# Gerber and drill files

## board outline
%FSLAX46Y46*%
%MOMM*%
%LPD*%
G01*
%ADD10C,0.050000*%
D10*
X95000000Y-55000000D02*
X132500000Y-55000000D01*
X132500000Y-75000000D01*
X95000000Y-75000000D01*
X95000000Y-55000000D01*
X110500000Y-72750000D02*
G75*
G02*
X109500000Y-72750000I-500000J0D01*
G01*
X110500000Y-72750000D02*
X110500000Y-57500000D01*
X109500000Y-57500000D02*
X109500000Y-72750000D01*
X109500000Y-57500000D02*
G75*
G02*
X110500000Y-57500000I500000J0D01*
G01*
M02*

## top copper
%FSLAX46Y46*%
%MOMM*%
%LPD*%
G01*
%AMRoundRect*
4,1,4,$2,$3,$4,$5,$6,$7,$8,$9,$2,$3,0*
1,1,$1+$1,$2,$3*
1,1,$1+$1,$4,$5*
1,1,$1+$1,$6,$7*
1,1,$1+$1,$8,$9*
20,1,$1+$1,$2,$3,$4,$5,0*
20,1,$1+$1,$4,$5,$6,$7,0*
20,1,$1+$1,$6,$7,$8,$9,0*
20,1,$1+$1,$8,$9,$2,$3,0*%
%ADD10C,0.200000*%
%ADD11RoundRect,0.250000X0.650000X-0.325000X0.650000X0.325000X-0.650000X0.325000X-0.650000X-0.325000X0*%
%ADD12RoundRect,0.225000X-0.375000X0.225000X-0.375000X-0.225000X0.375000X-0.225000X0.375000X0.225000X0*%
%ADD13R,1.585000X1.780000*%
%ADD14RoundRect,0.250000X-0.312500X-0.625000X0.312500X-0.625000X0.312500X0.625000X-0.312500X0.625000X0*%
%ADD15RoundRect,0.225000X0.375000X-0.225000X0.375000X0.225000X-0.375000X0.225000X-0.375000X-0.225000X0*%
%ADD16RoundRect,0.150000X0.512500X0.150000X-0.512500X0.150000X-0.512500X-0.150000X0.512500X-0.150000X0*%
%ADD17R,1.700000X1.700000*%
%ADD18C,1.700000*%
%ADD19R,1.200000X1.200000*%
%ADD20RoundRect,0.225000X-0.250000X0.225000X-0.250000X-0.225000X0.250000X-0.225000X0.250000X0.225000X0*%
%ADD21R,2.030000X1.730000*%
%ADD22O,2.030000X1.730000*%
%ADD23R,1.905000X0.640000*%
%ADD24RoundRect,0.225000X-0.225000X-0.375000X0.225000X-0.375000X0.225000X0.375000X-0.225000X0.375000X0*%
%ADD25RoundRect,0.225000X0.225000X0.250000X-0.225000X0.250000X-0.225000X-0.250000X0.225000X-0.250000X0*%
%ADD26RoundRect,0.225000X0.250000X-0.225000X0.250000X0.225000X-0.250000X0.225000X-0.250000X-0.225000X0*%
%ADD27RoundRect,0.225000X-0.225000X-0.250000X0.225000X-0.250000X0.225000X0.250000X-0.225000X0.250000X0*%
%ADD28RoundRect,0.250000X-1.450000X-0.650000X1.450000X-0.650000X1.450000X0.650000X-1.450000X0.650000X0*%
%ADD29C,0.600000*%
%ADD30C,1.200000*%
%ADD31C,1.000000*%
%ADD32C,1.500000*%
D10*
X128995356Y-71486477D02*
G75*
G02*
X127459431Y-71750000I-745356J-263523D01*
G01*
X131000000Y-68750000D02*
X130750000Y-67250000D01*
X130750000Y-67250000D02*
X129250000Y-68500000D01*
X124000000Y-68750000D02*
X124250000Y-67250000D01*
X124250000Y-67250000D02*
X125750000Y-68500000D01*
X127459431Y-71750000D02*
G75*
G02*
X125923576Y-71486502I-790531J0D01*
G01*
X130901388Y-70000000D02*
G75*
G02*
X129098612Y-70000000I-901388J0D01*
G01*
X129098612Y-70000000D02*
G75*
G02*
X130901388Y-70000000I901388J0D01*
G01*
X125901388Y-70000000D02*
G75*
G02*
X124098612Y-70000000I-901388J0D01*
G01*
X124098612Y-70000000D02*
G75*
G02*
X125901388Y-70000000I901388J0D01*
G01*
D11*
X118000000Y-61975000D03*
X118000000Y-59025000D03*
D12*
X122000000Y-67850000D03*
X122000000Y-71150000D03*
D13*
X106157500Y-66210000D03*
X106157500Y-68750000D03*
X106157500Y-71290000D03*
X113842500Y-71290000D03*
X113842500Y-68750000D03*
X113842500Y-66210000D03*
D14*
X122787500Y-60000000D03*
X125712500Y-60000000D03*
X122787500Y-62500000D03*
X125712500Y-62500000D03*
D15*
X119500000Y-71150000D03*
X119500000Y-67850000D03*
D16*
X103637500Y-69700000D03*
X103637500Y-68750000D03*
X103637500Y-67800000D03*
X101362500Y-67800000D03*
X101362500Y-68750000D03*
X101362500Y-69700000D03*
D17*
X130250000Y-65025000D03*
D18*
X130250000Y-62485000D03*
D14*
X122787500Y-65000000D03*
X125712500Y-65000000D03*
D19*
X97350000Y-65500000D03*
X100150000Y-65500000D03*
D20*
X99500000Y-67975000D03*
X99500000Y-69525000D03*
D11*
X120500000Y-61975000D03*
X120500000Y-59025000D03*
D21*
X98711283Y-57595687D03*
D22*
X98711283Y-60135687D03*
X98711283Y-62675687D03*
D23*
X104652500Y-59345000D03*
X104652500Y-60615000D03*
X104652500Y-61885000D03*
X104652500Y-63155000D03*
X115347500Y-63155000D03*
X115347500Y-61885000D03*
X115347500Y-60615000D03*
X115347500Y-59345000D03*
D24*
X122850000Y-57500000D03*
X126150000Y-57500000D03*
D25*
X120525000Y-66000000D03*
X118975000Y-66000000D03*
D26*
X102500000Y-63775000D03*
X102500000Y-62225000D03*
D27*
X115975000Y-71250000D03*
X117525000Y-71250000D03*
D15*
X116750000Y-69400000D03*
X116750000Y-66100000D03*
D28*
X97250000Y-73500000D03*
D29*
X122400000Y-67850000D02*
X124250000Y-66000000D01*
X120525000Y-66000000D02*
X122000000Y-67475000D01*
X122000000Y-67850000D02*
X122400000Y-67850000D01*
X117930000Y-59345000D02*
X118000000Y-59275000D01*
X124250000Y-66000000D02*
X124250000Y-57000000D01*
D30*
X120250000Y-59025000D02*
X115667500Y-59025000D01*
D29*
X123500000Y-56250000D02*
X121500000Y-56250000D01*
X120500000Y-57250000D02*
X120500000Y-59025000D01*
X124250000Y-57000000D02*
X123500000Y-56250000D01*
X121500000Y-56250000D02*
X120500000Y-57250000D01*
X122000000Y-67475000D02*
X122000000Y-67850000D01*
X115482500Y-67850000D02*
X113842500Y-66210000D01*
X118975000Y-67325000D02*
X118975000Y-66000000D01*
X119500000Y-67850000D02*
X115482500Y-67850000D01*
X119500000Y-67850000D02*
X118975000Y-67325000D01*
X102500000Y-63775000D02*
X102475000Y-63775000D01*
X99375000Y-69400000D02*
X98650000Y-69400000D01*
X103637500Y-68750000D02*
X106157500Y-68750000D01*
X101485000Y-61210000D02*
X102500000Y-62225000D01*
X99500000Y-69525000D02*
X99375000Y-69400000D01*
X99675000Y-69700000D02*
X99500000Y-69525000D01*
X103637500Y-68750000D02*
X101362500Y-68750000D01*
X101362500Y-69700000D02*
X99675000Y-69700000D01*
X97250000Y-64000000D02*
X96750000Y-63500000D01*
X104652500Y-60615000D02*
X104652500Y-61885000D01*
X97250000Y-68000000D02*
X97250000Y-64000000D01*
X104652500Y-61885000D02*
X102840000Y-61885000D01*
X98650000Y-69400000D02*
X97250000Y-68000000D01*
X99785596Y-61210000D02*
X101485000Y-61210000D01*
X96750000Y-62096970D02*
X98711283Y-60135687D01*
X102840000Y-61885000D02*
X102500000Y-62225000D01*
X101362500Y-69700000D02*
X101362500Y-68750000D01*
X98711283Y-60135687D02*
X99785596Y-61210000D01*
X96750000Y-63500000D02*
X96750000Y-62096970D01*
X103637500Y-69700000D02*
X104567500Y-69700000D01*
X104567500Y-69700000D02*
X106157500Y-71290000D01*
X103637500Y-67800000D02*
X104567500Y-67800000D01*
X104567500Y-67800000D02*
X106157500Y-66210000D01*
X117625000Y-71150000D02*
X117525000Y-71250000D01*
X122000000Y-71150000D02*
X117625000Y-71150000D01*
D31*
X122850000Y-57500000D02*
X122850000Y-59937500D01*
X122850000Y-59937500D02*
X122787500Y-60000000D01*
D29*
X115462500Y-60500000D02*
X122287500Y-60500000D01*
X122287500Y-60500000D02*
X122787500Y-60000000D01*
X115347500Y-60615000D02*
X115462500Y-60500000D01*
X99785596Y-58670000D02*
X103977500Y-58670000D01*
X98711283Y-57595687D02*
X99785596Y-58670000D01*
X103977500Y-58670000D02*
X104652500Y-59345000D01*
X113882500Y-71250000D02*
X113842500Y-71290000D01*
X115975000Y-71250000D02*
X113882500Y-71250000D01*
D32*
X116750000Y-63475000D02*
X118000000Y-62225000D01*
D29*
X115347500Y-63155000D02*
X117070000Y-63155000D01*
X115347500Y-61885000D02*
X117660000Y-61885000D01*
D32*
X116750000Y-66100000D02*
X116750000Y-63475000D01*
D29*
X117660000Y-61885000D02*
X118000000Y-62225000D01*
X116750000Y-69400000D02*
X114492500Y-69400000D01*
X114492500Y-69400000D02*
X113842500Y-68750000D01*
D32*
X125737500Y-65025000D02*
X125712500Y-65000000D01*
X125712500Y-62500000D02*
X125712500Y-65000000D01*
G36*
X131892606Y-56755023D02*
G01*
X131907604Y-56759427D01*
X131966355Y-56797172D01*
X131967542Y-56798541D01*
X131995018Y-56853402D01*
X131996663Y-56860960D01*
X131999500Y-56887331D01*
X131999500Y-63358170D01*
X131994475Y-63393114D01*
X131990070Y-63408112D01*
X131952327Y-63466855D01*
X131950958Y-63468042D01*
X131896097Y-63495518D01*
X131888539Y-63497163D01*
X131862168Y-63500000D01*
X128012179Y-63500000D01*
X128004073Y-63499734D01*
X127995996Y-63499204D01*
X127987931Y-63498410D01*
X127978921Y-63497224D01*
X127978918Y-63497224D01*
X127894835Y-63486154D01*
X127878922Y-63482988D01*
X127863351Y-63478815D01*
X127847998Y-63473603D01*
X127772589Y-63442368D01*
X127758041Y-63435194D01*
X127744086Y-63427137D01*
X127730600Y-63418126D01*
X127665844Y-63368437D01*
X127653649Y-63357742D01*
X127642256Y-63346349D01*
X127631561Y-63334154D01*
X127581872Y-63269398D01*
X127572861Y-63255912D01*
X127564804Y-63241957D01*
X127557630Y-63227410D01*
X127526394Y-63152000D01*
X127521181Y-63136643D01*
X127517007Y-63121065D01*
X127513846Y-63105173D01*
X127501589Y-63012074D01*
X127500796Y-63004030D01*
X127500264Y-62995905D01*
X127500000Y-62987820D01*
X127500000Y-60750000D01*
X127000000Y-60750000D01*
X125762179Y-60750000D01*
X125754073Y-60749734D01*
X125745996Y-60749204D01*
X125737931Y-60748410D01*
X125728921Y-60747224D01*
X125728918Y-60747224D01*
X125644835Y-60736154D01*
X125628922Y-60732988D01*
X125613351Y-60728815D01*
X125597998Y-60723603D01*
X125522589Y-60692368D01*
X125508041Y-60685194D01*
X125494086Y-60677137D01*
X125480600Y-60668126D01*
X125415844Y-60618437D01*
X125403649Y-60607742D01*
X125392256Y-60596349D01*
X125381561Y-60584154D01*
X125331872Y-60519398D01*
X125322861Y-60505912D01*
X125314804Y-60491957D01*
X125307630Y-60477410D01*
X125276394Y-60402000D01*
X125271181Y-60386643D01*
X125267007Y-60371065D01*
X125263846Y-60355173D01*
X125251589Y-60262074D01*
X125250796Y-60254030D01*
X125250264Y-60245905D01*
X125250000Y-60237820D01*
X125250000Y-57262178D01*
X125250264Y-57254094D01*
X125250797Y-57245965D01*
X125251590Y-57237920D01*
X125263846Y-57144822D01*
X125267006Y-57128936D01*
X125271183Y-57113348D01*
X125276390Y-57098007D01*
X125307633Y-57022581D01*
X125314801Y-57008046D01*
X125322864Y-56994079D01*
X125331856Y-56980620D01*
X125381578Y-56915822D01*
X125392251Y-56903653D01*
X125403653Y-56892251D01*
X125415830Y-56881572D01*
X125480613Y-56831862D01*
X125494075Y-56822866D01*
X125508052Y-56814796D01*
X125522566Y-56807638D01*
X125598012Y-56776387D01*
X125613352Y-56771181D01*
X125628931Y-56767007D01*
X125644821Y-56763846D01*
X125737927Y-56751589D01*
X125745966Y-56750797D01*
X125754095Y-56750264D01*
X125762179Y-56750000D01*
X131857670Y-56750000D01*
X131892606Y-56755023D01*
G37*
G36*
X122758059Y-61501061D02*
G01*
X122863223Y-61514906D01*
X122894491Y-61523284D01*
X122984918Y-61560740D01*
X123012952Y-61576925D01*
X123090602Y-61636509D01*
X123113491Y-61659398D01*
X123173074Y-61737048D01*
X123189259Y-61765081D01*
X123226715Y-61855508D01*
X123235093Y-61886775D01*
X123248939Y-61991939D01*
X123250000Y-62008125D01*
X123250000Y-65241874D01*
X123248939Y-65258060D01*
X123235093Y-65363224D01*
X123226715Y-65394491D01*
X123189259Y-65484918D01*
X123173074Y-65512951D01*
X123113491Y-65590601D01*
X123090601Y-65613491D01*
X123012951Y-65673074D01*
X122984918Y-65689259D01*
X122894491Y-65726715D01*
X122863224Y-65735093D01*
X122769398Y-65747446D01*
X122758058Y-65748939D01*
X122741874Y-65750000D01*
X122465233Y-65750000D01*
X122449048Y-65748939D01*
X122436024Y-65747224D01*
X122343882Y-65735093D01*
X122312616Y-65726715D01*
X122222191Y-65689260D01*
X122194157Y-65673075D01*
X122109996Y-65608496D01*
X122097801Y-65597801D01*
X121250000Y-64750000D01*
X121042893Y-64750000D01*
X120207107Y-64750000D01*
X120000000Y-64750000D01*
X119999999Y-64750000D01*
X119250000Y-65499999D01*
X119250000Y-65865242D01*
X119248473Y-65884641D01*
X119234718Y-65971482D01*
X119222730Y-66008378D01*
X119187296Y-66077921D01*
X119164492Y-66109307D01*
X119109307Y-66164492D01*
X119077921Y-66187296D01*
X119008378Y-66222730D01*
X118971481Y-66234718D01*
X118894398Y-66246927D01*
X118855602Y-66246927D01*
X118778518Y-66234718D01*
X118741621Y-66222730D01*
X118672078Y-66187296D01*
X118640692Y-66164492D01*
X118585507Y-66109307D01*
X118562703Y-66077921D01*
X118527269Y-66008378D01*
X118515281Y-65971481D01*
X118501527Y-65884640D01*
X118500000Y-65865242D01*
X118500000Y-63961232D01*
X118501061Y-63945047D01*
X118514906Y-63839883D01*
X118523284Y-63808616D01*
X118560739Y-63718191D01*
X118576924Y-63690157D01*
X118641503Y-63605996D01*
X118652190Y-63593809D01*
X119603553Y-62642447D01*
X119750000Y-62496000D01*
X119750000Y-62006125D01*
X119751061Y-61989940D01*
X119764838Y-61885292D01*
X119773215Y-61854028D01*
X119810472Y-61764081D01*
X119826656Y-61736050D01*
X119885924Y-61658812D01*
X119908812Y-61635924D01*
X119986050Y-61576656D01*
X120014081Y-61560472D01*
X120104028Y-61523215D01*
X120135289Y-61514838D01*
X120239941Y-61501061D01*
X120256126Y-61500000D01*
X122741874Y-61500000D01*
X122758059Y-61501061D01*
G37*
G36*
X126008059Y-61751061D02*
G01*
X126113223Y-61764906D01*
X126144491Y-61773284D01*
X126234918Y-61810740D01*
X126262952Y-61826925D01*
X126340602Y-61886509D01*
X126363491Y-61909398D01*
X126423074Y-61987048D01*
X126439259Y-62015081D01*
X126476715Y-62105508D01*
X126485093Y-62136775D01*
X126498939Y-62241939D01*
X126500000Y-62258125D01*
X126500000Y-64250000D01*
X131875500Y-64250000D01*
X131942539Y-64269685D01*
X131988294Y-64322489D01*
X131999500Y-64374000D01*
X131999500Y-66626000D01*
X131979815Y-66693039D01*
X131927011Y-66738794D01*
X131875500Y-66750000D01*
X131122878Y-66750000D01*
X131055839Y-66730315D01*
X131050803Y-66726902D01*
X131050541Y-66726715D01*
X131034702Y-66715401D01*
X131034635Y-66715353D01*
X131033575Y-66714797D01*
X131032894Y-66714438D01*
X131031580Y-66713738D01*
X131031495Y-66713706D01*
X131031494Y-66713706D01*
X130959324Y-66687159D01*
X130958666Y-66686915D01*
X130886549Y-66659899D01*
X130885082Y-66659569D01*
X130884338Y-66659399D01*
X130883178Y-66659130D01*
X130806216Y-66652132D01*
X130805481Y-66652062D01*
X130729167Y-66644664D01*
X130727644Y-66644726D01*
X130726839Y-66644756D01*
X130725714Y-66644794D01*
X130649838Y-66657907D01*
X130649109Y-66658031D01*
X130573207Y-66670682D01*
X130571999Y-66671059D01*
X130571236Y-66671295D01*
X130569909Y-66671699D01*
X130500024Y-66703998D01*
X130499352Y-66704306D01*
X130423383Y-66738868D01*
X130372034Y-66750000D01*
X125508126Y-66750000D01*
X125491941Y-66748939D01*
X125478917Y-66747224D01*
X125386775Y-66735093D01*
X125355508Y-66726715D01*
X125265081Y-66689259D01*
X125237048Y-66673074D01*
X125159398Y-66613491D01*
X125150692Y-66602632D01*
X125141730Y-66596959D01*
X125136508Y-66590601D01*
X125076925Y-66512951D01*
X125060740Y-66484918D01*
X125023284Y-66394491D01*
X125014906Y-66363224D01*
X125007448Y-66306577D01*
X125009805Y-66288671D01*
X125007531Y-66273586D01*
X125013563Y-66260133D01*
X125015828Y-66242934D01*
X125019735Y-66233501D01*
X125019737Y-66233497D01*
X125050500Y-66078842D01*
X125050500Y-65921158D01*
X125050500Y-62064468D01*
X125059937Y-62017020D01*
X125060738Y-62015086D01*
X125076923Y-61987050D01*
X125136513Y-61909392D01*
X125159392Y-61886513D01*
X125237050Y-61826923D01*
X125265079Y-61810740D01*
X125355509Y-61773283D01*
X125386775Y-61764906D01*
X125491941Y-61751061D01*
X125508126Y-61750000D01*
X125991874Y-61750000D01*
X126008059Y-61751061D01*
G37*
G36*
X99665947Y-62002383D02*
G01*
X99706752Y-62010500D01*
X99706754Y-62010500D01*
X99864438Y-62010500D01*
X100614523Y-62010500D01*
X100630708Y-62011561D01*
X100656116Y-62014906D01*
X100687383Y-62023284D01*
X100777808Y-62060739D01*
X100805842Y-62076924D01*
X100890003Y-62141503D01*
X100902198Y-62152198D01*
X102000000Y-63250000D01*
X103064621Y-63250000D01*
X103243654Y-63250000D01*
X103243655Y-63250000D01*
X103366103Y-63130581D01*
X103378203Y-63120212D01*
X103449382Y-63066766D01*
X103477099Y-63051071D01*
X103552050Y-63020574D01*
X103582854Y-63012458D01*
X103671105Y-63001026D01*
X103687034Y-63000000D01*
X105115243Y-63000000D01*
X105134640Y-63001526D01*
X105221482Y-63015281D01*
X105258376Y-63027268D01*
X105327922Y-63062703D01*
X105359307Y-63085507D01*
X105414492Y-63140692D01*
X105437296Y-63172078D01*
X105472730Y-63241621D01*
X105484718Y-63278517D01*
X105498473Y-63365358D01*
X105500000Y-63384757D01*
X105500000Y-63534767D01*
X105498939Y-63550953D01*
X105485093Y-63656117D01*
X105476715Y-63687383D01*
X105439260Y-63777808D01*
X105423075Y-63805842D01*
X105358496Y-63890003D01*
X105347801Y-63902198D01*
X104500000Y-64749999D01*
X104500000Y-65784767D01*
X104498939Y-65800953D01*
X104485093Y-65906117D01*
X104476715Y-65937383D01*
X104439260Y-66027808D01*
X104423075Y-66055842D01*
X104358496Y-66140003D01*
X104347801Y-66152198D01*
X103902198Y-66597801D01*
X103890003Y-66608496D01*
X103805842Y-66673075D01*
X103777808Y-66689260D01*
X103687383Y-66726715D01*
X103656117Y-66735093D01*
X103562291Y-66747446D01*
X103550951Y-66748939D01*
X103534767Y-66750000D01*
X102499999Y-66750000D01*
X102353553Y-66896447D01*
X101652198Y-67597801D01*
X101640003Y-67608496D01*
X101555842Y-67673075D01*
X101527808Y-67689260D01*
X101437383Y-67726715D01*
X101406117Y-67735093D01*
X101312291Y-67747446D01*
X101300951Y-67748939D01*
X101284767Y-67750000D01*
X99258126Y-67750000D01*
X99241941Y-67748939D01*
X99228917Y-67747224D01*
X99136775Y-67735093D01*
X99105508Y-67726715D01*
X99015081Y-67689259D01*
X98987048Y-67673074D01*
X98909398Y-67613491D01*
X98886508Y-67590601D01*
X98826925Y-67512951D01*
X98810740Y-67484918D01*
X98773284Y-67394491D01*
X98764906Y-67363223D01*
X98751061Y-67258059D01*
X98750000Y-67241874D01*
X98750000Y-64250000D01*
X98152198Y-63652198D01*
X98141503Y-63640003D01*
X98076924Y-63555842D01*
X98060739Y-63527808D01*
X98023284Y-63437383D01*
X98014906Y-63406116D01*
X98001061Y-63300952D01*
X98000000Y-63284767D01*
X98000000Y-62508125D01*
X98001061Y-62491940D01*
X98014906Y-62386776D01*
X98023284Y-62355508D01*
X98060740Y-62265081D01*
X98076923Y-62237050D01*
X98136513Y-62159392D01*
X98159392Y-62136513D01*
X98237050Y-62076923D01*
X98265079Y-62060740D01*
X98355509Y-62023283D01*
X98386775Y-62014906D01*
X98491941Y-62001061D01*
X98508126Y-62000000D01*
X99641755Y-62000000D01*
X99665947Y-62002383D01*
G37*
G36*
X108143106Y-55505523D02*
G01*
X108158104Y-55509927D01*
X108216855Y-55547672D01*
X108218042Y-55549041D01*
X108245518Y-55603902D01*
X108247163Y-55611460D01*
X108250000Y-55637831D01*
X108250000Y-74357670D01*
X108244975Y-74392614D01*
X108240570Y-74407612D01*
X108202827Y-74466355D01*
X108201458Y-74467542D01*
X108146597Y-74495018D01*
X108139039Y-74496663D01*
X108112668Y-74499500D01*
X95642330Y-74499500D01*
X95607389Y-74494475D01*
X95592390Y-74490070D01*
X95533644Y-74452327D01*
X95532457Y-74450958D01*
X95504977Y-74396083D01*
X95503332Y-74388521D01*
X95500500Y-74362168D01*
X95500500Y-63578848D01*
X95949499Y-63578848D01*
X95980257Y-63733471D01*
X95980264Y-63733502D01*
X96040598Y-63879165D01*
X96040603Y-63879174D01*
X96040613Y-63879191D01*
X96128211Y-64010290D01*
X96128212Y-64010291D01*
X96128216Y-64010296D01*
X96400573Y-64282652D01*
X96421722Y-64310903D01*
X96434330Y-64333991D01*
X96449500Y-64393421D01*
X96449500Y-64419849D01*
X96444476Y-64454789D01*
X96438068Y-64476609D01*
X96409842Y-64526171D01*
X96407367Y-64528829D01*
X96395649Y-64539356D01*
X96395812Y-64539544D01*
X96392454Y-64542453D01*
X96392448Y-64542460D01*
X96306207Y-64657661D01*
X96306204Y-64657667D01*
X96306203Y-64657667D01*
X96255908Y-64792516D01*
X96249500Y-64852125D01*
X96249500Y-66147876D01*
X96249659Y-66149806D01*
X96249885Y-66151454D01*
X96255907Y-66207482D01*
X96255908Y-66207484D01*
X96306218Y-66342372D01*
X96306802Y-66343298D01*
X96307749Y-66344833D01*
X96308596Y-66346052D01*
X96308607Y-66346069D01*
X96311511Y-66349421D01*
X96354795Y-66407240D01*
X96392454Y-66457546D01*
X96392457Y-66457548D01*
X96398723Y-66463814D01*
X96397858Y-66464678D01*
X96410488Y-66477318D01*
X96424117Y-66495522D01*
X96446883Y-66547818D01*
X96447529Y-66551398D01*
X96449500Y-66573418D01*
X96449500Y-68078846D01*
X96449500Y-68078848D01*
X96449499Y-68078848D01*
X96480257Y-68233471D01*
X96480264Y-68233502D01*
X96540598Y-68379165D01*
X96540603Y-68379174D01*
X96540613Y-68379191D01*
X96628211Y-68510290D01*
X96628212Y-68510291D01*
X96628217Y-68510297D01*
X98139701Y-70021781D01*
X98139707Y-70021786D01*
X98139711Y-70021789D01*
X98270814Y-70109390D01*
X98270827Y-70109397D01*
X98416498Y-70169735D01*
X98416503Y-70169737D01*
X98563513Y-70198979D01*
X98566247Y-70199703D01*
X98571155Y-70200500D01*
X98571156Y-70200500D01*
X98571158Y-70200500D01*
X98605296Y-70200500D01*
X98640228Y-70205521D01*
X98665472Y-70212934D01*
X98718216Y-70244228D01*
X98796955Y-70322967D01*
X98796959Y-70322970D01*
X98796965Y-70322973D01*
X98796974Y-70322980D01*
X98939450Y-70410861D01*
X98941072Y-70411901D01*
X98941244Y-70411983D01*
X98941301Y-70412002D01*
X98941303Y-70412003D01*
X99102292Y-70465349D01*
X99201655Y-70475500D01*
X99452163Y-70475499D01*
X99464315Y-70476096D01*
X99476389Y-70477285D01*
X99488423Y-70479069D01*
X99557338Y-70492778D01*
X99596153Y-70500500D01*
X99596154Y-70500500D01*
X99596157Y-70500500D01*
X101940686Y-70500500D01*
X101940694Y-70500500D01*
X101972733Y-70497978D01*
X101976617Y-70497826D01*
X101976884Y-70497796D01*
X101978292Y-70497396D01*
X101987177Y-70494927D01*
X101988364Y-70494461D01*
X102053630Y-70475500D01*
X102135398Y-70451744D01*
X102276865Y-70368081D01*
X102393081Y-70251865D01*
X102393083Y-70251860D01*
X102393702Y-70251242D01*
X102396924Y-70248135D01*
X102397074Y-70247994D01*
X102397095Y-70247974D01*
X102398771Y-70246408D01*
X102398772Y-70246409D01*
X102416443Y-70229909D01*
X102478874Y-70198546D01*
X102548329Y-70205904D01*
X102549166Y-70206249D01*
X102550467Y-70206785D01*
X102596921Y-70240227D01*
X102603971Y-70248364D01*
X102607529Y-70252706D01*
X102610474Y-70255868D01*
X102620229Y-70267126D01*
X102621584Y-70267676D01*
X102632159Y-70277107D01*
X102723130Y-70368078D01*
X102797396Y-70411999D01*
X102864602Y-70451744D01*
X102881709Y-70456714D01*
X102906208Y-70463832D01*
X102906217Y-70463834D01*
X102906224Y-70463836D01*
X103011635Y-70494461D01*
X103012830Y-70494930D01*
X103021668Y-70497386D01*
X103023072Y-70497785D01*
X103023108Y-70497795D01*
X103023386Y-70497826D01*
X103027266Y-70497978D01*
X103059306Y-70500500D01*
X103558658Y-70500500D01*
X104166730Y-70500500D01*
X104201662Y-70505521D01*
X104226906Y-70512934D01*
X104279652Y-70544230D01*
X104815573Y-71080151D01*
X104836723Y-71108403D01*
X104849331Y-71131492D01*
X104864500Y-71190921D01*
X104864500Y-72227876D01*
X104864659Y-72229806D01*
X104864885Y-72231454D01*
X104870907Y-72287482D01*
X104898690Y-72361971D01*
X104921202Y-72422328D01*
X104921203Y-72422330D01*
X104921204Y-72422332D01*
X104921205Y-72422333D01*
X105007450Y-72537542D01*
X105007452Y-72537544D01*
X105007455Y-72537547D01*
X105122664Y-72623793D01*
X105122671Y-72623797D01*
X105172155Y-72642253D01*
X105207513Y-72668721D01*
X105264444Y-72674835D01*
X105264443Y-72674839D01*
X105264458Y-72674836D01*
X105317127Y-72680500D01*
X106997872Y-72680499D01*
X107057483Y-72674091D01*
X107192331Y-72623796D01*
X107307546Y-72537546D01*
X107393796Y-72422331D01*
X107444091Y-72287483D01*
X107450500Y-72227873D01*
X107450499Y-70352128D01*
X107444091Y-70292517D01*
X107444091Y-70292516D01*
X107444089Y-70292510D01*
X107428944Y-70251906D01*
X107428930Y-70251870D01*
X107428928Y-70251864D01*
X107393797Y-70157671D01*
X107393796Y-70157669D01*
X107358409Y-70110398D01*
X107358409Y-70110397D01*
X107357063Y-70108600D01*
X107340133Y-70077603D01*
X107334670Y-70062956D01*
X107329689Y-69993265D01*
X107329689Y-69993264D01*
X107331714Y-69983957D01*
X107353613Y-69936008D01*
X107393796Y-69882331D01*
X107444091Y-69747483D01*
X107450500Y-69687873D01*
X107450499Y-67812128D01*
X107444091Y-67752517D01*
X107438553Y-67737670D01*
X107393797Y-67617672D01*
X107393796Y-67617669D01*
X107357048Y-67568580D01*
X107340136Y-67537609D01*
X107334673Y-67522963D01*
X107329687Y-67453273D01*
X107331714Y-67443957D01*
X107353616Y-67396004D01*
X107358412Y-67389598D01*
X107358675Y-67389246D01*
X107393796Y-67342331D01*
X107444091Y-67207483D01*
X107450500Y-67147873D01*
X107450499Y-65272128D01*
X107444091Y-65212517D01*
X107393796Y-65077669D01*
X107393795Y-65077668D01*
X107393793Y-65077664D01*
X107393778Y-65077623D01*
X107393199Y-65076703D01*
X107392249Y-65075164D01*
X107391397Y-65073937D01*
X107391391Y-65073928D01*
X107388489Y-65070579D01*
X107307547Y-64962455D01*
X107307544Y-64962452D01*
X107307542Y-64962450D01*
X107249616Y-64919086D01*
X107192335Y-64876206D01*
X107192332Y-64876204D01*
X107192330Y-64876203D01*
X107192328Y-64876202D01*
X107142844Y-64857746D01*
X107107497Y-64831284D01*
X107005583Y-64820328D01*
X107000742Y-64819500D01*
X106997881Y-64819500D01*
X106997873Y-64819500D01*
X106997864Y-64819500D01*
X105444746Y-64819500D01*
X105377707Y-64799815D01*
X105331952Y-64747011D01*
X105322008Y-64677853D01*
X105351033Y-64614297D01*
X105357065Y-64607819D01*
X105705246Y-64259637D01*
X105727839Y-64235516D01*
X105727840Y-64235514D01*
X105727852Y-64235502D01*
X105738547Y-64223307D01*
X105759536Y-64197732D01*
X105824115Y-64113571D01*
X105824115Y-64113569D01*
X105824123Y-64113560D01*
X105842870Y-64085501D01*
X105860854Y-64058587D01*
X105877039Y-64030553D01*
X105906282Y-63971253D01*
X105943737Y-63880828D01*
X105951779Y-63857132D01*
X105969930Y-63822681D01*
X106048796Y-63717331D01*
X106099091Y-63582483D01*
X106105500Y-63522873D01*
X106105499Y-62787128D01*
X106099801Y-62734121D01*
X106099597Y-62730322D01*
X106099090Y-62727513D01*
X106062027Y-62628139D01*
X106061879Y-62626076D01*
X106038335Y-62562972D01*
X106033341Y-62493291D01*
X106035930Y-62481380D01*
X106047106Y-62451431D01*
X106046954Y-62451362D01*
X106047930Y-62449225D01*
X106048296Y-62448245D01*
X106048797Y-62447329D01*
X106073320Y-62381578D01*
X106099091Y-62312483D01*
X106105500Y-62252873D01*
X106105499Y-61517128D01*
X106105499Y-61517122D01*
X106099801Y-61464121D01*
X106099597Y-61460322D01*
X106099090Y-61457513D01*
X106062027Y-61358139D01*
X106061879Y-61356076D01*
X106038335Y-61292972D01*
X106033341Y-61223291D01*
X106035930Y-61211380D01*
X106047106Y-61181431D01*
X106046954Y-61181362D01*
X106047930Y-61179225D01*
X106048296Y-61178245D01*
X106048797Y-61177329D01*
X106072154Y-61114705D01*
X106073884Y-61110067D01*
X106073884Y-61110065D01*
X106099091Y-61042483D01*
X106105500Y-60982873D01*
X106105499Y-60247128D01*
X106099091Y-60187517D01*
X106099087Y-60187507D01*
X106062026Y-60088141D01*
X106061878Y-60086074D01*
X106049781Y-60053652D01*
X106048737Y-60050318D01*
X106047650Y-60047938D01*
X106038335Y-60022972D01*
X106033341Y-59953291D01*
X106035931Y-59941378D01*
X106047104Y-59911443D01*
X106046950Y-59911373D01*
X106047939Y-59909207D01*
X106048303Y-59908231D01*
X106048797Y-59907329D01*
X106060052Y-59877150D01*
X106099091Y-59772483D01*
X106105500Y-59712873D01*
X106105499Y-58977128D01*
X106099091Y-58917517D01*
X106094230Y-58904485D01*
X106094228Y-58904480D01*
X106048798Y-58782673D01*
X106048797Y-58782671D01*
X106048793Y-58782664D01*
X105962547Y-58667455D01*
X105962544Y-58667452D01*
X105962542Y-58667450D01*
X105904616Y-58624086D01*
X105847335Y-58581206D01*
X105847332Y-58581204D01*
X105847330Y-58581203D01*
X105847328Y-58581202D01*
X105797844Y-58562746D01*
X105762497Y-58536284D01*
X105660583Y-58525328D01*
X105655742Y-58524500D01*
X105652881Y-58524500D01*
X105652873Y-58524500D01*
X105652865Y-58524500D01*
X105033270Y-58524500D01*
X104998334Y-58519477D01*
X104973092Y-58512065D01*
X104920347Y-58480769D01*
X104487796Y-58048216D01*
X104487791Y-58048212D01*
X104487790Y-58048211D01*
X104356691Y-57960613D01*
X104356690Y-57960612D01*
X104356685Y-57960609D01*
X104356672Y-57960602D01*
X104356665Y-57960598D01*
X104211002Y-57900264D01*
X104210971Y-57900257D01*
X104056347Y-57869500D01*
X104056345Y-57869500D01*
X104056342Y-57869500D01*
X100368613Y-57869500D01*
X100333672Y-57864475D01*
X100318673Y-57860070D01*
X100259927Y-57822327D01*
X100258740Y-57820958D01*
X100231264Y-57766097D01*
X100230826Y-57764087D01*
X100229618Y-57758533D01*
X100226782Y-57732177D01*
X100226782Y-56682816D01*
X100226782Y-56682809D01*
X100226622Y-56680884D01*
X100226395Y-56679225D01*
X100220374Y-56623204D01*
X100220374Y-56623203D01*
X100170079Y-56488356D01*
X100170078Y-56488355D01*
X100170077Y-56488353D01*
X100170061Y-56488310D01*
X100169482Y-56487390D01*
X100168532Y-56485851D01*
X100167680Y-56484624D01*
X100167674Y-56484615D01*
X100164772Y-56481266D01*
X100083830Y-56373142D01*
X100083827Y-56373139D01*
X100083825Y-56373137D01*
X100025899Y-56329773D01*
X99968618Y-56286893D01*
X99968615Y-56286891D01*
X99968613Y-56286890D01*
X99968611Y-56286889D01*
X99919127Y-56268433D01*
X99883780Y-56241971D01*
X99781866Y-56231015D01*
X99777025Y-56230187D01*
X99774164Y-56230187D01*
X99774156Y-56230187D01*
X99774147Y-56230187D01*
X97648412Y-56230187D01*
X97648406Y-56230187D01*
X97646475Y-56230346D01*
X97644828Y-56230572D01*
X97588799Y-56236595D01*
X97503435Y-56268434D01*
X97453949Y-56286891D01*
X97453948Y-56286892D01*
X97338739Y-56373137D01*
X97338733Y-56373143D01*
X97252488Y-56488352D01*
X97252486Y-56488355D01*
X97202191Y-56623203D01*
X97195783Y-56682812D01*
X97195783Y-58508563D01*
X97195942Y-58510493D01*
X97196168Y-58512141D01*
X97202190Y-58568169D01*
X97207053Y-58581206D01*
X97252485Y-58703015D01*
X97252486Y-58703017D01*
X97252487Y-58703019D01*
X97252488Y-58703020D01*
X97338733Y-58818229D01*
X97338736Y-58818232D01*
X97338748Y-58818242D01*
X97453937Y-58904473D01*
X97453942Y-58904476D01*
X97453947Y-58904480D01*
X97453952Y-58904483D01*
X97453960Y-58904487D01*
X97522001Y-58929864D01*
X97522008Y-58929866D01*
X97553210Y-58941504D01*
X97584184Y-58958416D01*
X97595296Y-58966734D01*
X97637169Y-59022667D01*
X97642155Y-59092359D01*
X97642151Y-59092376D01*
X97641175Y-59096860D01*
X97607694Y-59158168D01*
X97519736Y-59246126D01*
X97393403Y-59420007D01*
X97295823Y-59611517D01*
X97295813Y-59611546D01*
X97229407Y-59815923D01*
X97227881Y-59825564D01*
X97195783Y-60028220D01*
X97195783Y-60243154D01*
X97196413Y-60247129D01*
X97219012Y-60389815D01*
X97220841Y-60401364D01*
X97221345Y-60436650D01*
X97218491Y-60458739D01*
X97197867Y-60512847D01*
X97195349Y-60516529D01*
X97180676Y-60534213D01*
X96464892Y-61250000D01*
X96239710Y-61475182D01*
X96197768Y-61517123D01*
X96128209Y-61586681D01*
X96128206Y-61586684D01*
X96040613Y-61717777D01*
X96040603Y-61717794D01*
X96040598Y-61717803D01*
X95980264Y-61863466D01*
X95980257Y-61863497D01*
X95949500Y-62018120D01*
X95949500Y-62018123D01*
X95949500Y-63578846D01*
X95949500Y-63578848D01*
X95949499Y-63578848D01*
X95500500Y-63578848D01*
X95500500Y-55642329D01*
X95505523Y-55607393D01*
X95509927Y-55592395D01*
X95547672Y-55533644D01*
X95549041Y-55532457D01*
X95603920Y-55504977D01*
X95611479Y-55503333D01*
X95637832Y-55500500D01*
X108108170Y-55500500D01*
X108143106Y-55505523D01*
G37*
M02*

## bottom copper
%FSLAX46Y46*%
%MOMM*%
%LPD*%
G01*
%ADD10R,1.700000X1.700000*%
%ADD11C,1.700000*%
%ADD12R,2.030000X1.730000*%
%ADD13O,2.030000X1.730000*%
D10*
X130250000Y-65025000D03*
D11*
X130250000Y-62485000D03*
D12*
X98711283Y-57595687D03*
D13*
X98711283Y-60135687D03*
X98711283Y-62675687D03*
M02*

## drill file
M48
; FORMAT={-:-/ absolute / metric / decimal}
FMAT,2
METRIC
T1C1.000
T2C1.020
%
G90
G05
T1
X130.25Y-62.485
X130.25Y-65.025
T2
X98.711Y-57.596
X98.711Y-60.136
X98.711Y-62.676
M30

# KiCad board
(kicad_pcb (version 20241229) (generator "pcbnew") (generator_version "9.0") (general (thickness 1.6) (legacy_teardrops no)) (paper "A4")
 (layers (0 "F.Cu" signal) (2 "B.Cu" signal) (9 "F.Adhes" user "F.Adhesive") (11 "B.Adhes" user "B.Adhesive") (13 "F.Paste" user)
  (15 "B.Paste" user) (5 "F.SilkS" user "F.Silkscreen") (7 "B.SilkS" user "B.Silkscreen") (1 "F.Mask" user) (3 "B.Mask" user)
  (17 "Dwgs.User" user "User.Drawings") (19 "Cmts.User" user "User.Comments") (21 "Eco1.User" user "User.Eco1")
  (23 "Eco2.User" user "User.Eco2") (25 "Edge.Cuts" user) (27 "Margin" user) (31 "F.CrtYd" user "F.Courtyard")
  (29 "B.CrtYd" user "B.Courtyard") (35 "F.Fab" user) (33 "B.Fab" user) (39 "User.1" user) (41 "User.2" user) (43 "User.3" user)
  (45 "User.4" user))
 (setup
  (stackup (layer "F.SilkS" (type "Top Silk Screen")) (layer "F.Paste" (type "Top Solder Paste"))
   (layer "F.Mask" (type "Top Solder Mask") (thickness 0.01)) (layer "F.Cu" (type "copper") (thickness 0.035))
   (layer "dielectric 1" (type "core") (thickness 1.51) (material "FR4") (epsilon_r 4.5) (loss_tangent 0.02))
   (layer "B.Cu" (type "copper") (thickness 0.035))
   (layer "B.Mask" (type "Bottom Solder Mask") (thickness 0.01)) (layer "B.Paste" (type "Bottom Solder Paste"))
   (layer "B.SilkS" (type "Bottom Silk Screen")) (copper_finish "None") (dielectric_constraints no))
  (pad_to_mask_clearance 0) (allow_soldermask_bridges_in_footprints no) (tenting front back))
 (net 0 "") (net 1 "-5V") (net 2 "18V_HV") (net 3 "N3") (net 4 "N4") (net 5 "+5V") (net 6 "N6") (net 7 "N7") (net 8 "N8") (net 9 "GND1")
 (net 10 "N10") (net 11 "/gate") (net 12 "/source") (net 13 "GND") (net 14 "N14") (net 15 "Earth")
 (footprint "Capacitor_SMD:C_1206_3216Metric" (layer "F.Cu") (at 118 60.5 90)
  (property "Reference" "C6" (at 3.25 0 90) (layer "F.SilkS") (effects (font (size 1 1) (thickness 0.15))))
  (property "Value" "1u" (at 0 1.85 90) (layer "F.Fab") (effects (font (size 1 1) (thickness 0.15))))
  (pad "1" smd roundrect (at -1.475 0 90) (size 1.15 1.8) (layers "F.Cu" "F.Mask" "F.Paste") (roundrect_rratio 0.217391) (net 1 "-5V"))
  (pad "2" smd roundrect (at 1.475 0 90) (size 1.15 1.8) (layers "F.Cu" "F.Mask" "F.Paste") (roundrect_rratio 0.217391) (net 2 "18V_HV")))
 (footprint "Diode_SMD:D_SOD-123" (layer "F.Cu") (at 122 69.5 -90)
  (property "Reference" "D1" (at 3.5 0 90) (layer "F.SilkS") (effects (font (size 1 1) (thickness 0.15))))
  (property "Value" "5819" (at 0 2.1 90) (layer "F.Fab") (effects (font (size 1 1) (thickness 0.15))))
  (pad "1" smd roundrect (at -1.65 0 270) (size 0.9 1.2) (layers "F.Cu" "F.Mask" "F.Paste") (roundrect_rratio 0.25) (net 2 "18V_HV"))
  (pad "2" smd roundrect (at 1.65 0 270) (size 0.9 1.2) (layers "F.Cu" "F.Mask" "F.Paste") (roundrect_rratio 0.25) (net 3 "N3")))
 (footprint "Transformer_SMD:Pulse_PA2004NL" (layer "F.Cu") (at 110 68.75)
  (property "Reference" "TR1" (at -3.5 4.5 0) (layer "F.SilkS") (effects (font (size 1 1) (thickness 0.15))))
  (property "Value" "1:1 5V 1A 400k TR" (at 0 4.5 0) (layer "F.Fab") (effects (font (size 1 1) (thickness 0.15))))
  (pad "1" smd rect (at -3.8425 -2.54) (size 1.585 1.78) (layers "F.Cu" "F.Mask" "F.Paste") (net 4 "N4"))
  (pad "2" smd rect (at -3.8425 0) (size 1.585 1.78) (layers "F.Cu" "F.Mask" "F.Paste") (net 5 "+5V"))
  (pad "3" smd rect (at -3.8425 2.54) (size 1.585 1.78) (layers "F.Cu" "F.Mask" "F.Paste") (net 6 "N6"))
  (pad "4" smd rect (at 3.8425 2.54) (size 1.585 1.78) (layers "F.Cu" "F.Mask" "F.Paste") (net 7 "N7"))
  (pad "5" smd rect (at 3.8425 0) (size 1.585 1.78) (layers "F.Cu" "F.Mask" "F.Paste") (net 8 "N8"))
  (pad "6" smd rect (at 3.8425 -2.54) (size 1.585 1.78) (layers "F.Cu" "F.Mask" "F.Paste") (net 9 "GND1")))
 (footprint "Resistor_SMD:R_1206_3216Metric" (layer "F.Cu") (at 124.25 60)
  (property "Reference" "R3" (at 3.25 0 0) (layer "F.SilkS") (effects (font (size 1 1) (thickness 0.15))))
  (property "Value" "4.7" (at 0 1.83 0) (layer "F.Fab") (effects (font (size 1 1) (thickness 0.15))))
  (pad "1" smd roundrect (at -1.4625 0) (size 1.125 1.75) (layers "F.Cu" "F.Mask" "F.Paste") (roundrect_rratio 0.222222) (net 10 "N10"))
  (pad "2" smd roundrect (at 1.4625 0) (size 1.125 1.75) (layers "F.Cu" "F.Mask" "F.Paste") (roundrect_rratio 0.222222) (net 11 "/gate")))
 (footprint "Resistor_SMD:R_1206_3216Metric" (layer "F.Cu") (at 124.25 62.5)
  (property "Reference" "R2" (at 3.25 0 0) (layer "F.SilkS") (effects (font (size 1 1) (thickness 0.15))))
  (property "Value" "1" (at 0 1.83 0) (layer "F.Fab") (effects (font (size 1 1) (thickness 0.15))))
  (pad "1" smd roundrect (at -1.4625 0) (size 1.125 1.75) (layers "F.Cu" "F.Mask" "F.Paste") (roundrect_rratio 0.222222) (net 9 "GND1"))
  (pad "2" smd roundrect (at 1.4625 0) (size 1.125 1.75) (layers "F.Cu" "F.Mask" "F.Paste") (roundrect_rratio 0.222222) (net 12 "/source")))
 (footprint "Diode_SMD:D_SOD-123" (layer "F.Cu") (at 119.5 69.5 90)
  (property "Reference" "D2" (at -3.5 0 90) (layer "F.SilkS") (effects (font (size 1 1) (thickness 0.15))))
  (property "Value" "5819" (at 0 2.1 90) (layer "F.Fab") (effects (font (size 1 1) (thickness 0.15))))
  (pad "1" smd roundrect (at -1.65 0 90) (size 0.9 1.2) (layers "F.Cu" "F.Mask" "F.Paste") (roundrect_rratio 0.25) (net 3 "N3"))
  (pad "2" smd roundrect (at 1.65 0 90) (size 0.9 1.2) (layers "F.Cu" "F.Mask" "F.Paste") (roundrect_rratio 0.25) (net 9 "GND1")))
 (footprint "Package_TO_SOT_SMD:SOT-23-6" (layer "F.Cu") (at 102.5 68.75 180)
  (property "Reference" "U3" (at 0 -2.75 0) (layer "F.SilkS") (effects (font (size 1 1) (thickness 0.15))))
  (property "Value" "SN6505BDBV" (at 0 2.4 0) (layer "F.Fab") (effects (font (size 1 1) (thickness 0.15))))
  (pad "1" smd roundrect (at -1.1375 -0.95 180) (size 1.325 0.6) (layers "F.Cu" "F.Mask" "F.Paste") (roundrect_rratio 0.25) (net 6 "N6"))
  (pad "2" smd roundrect (at -1.1375 0 180) (size 1.325 0.6) (layers "F.Cu" "F.Mask" "F.Paste") (roundrect_rratio 0.25) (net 5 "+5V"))
  (pad "3" smd roundrect (at -1.1375 0.95 180) (size 1.325 0.6) (layers "F.Cu" "F.Mask" "F.Paste") (roundrect_rratio 0.25) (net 4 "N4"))
  (pad "4" smd roundrect (at 1.1375 0.95 180) (size 1.325 0.6) (layers "F.Cu" "F.Mask" "F.Paste") (roundrect_rratio 0.25) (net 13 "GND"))
  (pad "5" smd roundrect (at 1.1375 0 180) (size 1.325 0.6) (layers "F.Cu" "F.Mask" "F.Paste") (roundrect_rratio 0.25) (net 5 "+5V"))
  (pad "6" smd roundrect (at 1.1375 -0.95 180) (size 1.325 0.6) (layers "F.Cu" "F.Mask" "F.Paste") (roundrect_rratio 0.25) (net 5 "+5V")))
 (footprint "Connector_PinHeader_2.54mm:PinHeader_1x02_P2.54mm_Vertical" (layer "F.Cu") (at 130.25 65.025 180)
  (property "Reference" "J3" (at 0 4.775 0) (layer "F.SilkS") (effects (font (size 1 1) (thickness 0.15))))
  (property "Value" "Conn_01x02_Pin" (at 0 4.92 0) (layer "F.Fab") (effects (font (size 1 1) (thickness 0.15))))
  (pad "1" thru_hole rect (at 0 0 180) (size 1.7 1.7) (drill 1) (layers "*.Cu" "*.Mask") (remove_unused_layers no) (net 12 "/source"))
  (pad "2" thru_hole circle (at 0 2.54 180) (size 1.7 1.7) (drill 1) (layers "*.Cu" "*.Mask") (remove_unused_layers no) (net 11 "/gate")))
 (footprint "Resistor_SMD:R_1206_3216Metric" (layer "F.Cu") (at 124.25 65)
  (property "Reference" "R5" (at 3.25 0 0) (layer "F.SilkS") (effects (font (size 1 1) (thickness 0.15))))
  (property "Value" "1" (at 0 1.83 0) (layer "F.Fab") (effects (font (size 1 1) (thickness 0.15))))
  (pad "1" smd roundrect (at -1.4625 0) (size 1.125 1.75) (layers "F.Cu" "F.Mask" "F.Paste") (roundrect_rratio 0.222222) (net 9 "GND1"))
  (pad "2" smd roundrect (at 1.4625 0) (size 1.125 1.75) (layers "F.Cu" "F.Mask" "F.Paste") (roundrect_rratio 0.222222) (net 12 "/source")))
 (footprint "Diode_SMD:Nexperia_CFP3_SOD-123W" (layer "F.Cu") (at 98.75 65.5)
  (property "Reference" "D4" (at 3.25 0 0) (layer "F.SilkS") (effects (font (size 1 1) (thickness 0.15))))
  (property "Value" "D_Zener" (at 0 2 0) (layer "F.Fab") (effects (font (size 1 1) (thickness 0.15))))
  (pad "1" smd rect (at -1.4 0) (size 1.2 1.2) (layers "F.Cu" "F.Mask" "F.Paste") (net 5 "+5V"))
  (pad "2" smd rect (at 1.4 0) (size 1.2 1.2) (layers "F.Cu" "F.Mask" "F.Paste") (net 13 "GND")))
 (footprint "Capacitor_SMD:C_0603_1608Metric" (layer "F.Cu") (at 99.5 68.75 -90)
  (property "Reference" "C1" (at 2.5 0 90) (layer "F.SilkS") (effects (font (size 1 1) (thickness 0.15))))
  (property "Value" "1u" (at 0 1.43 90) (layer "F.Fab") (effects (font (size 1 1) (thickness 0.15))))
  (pad "1" smd roundrect (at -0.775 0 270) (size 0.9 0.95) (layers "F.Cu" "F.Mask" "F.Paste") (roundrect_rratio 0.25) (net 13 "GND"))
  (pad "2" smd roundrect (at 0.775 0 270) (size 0.9 0.95) (layers "F.Cu" "F.Mask" "F.Paste") (roundrect_rratio 0.25) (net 5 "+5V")))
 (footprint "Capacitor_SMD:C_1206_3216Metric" (layer "F.Cu") (at 120.5 60.5 90)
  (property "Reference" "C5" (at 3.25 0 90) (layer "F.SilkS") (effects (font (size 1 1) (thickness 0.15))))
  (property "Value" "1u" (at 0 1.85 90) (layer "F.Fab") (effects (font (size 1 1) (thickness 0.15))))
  (pad "1" smd roundrect (at -1.475 0 90) (size 1.15 1.8) (layers "F.Cu" "F.Mask" "F.Paste") (roundrect_rratio 0.217391) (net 9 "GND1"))
  (pad "2" smd roundrect (at 1.475 0 90) (size 1.15 1.8) (layers "F.Cu" "F.Mask" "F.Paste") (roundrect_rratio 0.217391) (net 2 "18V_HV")))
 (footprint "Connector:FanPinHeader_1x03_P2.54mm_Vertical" (layer "F.Cu") (at 98.711283 57.595687 -90)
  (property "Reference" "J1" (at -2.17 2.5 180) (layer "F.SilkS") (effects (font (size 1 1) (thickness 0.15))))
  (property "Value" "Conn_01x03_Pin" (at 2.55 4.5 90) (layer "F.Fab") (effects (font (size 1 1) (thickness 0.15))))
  (pad "1" thru_hole rect (at 0 0) (size 2.03 1.73) (drill 1.02) (layers "*.Cu" "*.Mask") (remove_unused_layers no) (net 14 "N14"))
  (pad "2" thru_hole oval (at 2.54 0) (size 2.03 1.73) (drill 1.02) (layers "*.Cu" "*.Mask") (remove_unused_layers no) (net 5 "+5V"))
  (pad "3" thru_hole oval (at 5.08 0) (size 2.03 1.73) (drill 1.02) (layers "*.Cu" "*.Mask") (remove_unused_layers no) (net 13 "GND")))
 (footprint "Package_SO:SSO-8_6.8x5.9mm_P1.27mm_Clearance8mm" (layer "F.Cu") (at 110 61.25)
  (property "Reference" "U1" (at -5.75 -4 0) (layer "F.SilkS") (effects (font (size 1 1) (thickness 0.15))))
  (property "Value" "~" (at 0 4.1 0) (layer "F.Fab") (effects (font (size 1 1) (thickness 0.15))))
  (pad "1" smd rect (at -5.3475 -1.905) (size 1.905 0.64) (layers "F.Cu" "F.Mask" "F.Paste") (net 14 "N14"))
  (pad "2" smd rect (at -5.3475 -0.635) (size 1.905 0.64) (layers "F.Cu" "F.Mask" "F.Paste") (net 5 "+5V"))
  (pad "3" smd rect (at -5.3475 0.635) (size 1.905 0.64) (layers "F.Cu" "F.Mask" "F.Paste") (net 5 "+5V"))
  (pad "4" smd rect (at -5.3475 1.905) (size 1.905 0.64) (layers "F.Cu" "F.Mask" "F.Paste") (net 13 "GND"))
  (pad "5" smd rect (at 5.3475 1.905) (size 1.905 0.64) (layers "F.Cu" "F.Mask" "F.Paste") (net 1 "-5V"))
  (pad "6" smd rect (at 5.3475 0.635) (size 1.905 0.64) (layers "F.Cu" "F.Mask" "F.Paste") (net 1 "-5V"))
  (pad "7" smd rect (at 5.3475 -0.635) (size 1.905 0.64) (layers "F.Cu" "F.Mask" "F.Paste") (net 10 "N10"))
  (pad "8" smd rect (at 5.3475 -1.905) (size 1.905 0.64) (layers "F.Cu" "F.Mask" "F.Paste") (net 2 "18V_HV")))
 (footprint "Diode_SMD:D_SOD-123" (layer "F.Cu") (at 124.5 57.5)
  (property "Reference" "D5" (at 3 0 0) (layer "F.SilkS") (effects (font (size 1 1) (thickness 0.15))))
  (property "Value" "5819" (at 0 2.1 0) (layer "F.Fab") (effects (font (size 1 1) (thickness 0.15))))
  (pad "1" smd roundrect (at -1.65 0) (size 0.9 1.2) (layers "F.Cu" "F.Mask" "F.Paste") (roundrect_rratio 0.25) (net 10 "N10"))
  (pad "2" smd roundrect (at 1.65 0) (size 0.9 1.2) (layers "F.Cu" "F.Mask" "F.Paste") (roundrect_rratio 0.25) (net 11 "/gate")))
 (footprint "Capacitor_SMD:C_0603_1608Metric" (layer "F.Cu") (at 119.75 66 180)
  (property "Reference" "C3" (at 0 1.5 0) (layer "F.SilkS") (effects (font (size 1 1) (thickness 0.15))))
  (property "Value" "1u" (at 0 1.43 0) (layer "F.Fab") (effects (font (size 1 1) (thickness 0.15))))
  (pad "1" smd roundrect (at -0.775 0 180) (size 0.9 0.95) (layers "F.Cu" "F.Mask" "F.Paste") (roundrect_rratio 0.25) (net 2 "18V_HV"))
  (pad "2" smd roundrect (at 0.775 0 180) (size 0.9 0.95) (layers "F.Cu" "F.Mask" "F.Paste") (roundrect_rratio 0.25) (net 9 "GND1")))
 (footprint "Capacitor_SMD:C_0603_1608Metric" (layer "F.Cu") (at 102.5 63 90)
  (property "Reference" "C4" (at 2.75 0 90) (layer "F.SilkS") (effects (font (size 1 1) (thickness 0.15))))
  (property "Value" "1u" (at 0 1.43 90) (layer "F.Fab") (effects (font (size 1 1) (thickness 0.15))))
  (pad "1" smd roundrect (at -0.775 0 90) (size 0.9 0.95) (layers "F.Cu" "F.Mask" "F.Paste") (roundrect_rratio 0.25) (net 13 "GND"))
  (pad "2" smd roundrect (at 0.775 0 90) (size 0.9 0.95) (layers "F.Cu" "F.Mask" "F.Paste") (roundrect_rratio 0.25) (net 5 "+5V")))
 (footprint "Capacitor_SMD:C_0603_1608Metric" (layer "F.Cu") (at 116.75 71.25)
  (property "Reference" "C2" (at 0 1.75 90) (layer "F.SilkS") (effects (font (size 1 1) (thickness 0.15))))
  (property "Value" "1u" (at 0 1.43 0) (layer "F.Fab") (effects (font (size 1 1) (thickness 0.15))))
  (pad "1" smd roundrect (at -0.775 0) (size 0.9 0.95) (layers "F.Cu" "F.Mask" "F.Paste") (roundrect_rratio 0.25) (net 7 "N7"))
  (pad "2" smd roundrect (at 0.775 0) (size 0.9 0.95) (layers "F.Cu" "F.Mask" "F.Paste") (roundrect_rratio 0.25) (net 3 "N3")))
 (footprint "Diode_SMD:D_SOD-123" (layer "F.Cu") (at 116.75 67.75 90)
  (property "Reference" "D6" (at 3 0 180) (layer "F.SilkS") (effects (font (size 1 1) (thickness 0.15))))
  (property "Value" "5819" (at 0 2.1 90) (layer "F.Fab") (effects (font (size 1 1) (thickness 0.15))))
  (pad "1" smd roundrect (at -1.65 0 90) (size 0.9 1.2) (layers "F.Cu" "F.Mask" "F.Paste") (roundrect_rratio 0.25) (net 8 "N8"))
  (pad "2" smd roundrect (at 1.65 0 90) (size 0.9 1.2) (layers "F.Cu" "F.Mask" "F.Paste") (roundrect_rratio 0.25) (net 1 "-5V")))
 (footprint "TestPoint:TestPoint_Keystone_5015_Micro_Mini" (layer "F.Cu") (at 97.25 73.5)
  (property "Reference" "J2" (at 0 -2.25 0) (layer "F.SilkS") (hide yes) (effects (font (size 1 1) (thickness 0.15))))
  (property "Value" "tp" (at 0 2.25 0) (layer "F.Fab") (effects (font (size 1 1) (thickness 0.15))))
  (pad "1" smd roundrect (at 0 0) (size 3.4 1.8) (layers "F.Cu" "F.Mask" "F.Paste") (roundrect_rratio 0.1388888889) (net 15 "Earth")))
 (gr_arc (start 128.995356 71.486477) (mid 128.383687 72.529184) (end 127.459431 71.75) (stroke (width 0.2) (type default)) (layer "F.Cu"))
 (gr_line (start 131 68.75) (end 130.75 67.25) (stroke (width 0.2) (type default)) (layer "F.Cu"))
 (gr_line (start 130.75 67.25) (end 129.25 68.5) (stroke (width 0.2) (type default)) (layer "F.Cu"))
 (gr_line (start 124 68.75) (end 124.25 67.25) (stroke (width 0.2) (type default)) (layer "F.Cu"))
 (gr_line (start 124.25 67.25) (end 125.75 68.5) (stroke (width 0.2) (type default)) (layer "F.Cu"))
 (gr_arc (start 127.459431 71.75) (mid 126.535175 72.529184) (end 125.923506 71.486477) (stroke (width 0.2) (type default)) (layer "F.Cu"))
 (gr_circle (center 130 70) (end 130.75 70.5) (stroke (width 0.2) (type default)) (fill no) (layer "F.Cu"))
 (gr_circle (center 125 70) (end 125.75 70.5) (stroke (width 0.2) (type default)) (fill no) (layer "F.Cu"))
 (gr_rect (start 95 55) (end 132.5 75) (stroke (width 0.05) (type default)) (fill no) (layer "Edge.Cuts"))
 (gr_arc (start 110.5 72.75) (mid 110 73.25) (end 109.5 72.75) (stroke (width 0.05) (type default)) (layer "Edge.Cuts"))
 (gr_line (start 110.5 72.75) (end 110.5 57.5) (stroke (width 0.05) (type default)) (layer "Edge.Cuts"))
 (gr_line (start 109.5 57.5) (end 109.5 72.75) (stroke (width 0.05) (type default)) (layer "Edge.Cuts"))
 (gr_arc (start 109.5 57.5) (mid 110 57) (end 110.5 57.5) (stroke (width 0.05) (type default)) (layer "Edge.Cuts"))
 (segment (start 122.4 67.85) (end 124.25 66) (width 0.6) (layer "F.Cu") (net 2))
 (segment (start 120.525 66) (end 122 67.475) (width 0.6) (layer "F.Cu") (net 2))
 (segment (start 122 67.85) (end 122.4 67.85) (width 0.6) (layer "F.Cu") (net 2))
 (segment (start 117.93 59.345) (end 118 59.275) (width 0.6) (layer "F.Cu") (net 2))
 (segment (start 124.25 66) (end 124.25 57) (width 0.6) (layer "F.Cu") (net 2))
 (segment (start 120.25 59.025) (end 115.6675 59.025) (width 1.2) (layer "F.Cu") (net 2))
 (segment (start 123.5 56.25) (end 121.5 56.25) (width 0.6) (layer "F.Cu") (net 2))
 (segment (start 120.5 57.25) (end 120.5 59.025) (width 0.6) (layer "F.Cu") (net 2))
 (segment (start 124.25 57) (end 123.5 56.25) (width 0.6) (layer "F.Cu") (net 2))
 (segment (start 121.5 56.25) (end 120.5 57.25) (width 0.6) (layer "F.Cu") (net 2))
 (segment (start 122 67.475) (end 122 67.85) (width 0.6) (layer "F.Cu") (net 2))
 (segment (start 115.4825 67.85) (end 113.8425 66.21) (width 0.6) (layer "F.Cu") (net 9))
 (segment (start 118.975 67.325) (end 118.975 66) (width 0.6) (layer "F.Cu") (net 9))
 (segment (start 119.5 67.85) (end 115.4825 67.85) (width 0.6) (layer "F.Cu") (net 9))
 (segment (start 119.5 67.85) (end 118.975 67.325) (width 0.6) (layer "F.Cu") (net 9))
 (segment (start 102.5 63.775) (end 102.475 63.775) (width 0.6) (layer "F.Cu") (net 13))
 (segment (start 99.375 69.4) (end 98.65 69.4) (width 0.6) (layer "F.Cu") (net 5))
 (segment (start 103.6375 68.75) (end 106.1575 68.75) (width 0.6) (layer "F.Cu") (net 5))
 (segment (start 101.485 61.21) (end 102.5 62.225) (width 0.6) (layer "F.Cu") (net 5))
 (segment (start 99.5 69.525) (end 99.375 69.4) (width 0.6) (layer "F.Cu") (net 5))
 (segment (start 99.675 69.7) (end 99.5 69.525) (width 0.6) (layer "F.Cu") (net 5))
 (segment (start 103.6375 68.75) (end 101.3625 68.75) (width 0.6) (layer "F.Cu") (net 5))
 (segment (start 101.3625 69.7) (end 99.675 69.7) (width 0.6) (layer "F.Cu") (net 5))
 (segment (start 97.25 64) (end 96.75 63.5) (width 0.6) (layer "F.Cu") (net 5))
 (segment (start 104.6525 60.615) (end 104.6525 61.885) (width 0.6) (layer "F.Cu") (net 5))
 (segment (start 97.25 68) (end 97.25 64) (width 0.6) (layer "F.Cu") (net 5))
 (segment (start 104.6525 61.885) (end 102.84 61.885) (width 0.6) (layer "F.Cu") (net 5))
 (segment (start 98.65 69.4) (end 97.25 68) (width 0.6) (layer "F.Cu") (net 5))
 (segment (start 99.785596 61.21) (end 101.485 61.21) (width 0.6) (layer "F.Cu") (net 5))
 (segment (start 96.75 62.09697) (end 98.711283 60.135687) (width 0.6) (layer "F.Cu") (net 5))
 (segment (start 102.84 61.885) (end 102.5 62.225) (width 0.6) (layer "F.Cu") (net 5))
 (segment (start 101.3625 69.7) (end 101.3625 68.75) (width 0.6) (layer "F.Cu") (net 5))
 (segment (start 98.711283 60.135687) (end 99.785596 61.21) (width 0.6) (layer "F.Cu") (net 5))
 (segment (start 96.75 63.5) (end 96.75 62.09697) (width 0.6) (layer "F.Cu") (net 5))
 (segment (start 103.6375 69.7) (end 104.5675 69.7) (width 0.6) (layer "F.Cu") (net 6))
 (segment (start 104.5675 69.7) (end 106.1575 71.29) (width 0.6) (layer "F.Cu") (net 6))
 (segment (start 103.6375 67.8) (end 104.5675 67.8) (width 0.6) (layer "F.Cu") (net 4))
 (segment (start 104.5675 67.8) (end 106.1575 66.21) (width 0.6) (layer "F.Cu") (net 4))
 (segment (start 117.625 71.15) (end 117.525 71.25) (width 0.6) (layer "F.Cu") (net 3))
 (segment (start 122 71.15) (end 117.625 71.15) (width 0.6) (layer "F.Cu") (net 3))
 (segment (start 122.85 57.5) (end 122.85 59.9375) (width 1) (layer "F.Cu") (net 10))
 (segment (start 122.85 59.9375) (end 122.7875 60) (width 1) (layer "F.Cu") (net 10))
 (segment (start 115.4625 60.5) (end 122.2875 60.5) (width 0.6) (layer "F.Cu") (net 10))
 (segment (start 122.2875 60.5) (end 122.7875 60) (width 0.6) (layer "F.Cu") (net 10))
 (segment (start 115.3475 60.615) (end 115.4625 60.5) (width 0.6) (layer "F.Cu") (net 10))
 (segment (start 99.785596 58.67) (end 103.9775 58.67) (width 0.6) (layer "F.Cu") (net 14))
 (segment (start 98.711283 57.595687) (end 99.785596 58.67) (width 0.6) (layer "F.Cu") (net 14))
 (segment (start 103.9775 58.67) (end 104.6525 59.345) (width 0.6) (layer "F.Cu") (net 14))
 (segment (start 113.8825 71.25) (end 113.8425 71.29) (width 0.6) (layer "F.Cu") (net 7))
 (segment (start 115.975 71.25) (end 113.8825 71.25) (width 0.6) (layer "F.Cu") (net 7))
 (segment (start 116.75 63.475) (end 118 62.225) (width 1.5) (layer "F.Cu") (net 1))
 (segment (start 115.3475 63.155) (end 117.07 63.155) (width 0.6) (layer "F.Cu") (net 1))
 (segment (start 115.3475 61.885) (end 117.66 61.885) (width 0.6) (layer "F.Cu") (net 1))
 (segment (start 116.75 66.1) (end 116.75 63.475) (width 1.5) (layer "F.Cu") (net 1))
 (segment (start 117.66 61.885) (end 118 62.225) (width 0.6) (layer "F.Cu") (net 1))
 (segment (start 116.75 69.4) (end 114.4925 69.4) (width 0.6) (layer "F.Cu") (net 8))
 (segment (start 114.4925 69.4) (end 113.8425 68.75) (width 0.6) (layer "F.Cu") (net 8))
 (segment (start 125.7375 65.025) (end 125.7125 65) (width 1.5) (layer "F.Cu") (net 12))
 (segment (start 125.7125 62.5) (end 125.7125 65) (width 1.5) (layer "F.Cu") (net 12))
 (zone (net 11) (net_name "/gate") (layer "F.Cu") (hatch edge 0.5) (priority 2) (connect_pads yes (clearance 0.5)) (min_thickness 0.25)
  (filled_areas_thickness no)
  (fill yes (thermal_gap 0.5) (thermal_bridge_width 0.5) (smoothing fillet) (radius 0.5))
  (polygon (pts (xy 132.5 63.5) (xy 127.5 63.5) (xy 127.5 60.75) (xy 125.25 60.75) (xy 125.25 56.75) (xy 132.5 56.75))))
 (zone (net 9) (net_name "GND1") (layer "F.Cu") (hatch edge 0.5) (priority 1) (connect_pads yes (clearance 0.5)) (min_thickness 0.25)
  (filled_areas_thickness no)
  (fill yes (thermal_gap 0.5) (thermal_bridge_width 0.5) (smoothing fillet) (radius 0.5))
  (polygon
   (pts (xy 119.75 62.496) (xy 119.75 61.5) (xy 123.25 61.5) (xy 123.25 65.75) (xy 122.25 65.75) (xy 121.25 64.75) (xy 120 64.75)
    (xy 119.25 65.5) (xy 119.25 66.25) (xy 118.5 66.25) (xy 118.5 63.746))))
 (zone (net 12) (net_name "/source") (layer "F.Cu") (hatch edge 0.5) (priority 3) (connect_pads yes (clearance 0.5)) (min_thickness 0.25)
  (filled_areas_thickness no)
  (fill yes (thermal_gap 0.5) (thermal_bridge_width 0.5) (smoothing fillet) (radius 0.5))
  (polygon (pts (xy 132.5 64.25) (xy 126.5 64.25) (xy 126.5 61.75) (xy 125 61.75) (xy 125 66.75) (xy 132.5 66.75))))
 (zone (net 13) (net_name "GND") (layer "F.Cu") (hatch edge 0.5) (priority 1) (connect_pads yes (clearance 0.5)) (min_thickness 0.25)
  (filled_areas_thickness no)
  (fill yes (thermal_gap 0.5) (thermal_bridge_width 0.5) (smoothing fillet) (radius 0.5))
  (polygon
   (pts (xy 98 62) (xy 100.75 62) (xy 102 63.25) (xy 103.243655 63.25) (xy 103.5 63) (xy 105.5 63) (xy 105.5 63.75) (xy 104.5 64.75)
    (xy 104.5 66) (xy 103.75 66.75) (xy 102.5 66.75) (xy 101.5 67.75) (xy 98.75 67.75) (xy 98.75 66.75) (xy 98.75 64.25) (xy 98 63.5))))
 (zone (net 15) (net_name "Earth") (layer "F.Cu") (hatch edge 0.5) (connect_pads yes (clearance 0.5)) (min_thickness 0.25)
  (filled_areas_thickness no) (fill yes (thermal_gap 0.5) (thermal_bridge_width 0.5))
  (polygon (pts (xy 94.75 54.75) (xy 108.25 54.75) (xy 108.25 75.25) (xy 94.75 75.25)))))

